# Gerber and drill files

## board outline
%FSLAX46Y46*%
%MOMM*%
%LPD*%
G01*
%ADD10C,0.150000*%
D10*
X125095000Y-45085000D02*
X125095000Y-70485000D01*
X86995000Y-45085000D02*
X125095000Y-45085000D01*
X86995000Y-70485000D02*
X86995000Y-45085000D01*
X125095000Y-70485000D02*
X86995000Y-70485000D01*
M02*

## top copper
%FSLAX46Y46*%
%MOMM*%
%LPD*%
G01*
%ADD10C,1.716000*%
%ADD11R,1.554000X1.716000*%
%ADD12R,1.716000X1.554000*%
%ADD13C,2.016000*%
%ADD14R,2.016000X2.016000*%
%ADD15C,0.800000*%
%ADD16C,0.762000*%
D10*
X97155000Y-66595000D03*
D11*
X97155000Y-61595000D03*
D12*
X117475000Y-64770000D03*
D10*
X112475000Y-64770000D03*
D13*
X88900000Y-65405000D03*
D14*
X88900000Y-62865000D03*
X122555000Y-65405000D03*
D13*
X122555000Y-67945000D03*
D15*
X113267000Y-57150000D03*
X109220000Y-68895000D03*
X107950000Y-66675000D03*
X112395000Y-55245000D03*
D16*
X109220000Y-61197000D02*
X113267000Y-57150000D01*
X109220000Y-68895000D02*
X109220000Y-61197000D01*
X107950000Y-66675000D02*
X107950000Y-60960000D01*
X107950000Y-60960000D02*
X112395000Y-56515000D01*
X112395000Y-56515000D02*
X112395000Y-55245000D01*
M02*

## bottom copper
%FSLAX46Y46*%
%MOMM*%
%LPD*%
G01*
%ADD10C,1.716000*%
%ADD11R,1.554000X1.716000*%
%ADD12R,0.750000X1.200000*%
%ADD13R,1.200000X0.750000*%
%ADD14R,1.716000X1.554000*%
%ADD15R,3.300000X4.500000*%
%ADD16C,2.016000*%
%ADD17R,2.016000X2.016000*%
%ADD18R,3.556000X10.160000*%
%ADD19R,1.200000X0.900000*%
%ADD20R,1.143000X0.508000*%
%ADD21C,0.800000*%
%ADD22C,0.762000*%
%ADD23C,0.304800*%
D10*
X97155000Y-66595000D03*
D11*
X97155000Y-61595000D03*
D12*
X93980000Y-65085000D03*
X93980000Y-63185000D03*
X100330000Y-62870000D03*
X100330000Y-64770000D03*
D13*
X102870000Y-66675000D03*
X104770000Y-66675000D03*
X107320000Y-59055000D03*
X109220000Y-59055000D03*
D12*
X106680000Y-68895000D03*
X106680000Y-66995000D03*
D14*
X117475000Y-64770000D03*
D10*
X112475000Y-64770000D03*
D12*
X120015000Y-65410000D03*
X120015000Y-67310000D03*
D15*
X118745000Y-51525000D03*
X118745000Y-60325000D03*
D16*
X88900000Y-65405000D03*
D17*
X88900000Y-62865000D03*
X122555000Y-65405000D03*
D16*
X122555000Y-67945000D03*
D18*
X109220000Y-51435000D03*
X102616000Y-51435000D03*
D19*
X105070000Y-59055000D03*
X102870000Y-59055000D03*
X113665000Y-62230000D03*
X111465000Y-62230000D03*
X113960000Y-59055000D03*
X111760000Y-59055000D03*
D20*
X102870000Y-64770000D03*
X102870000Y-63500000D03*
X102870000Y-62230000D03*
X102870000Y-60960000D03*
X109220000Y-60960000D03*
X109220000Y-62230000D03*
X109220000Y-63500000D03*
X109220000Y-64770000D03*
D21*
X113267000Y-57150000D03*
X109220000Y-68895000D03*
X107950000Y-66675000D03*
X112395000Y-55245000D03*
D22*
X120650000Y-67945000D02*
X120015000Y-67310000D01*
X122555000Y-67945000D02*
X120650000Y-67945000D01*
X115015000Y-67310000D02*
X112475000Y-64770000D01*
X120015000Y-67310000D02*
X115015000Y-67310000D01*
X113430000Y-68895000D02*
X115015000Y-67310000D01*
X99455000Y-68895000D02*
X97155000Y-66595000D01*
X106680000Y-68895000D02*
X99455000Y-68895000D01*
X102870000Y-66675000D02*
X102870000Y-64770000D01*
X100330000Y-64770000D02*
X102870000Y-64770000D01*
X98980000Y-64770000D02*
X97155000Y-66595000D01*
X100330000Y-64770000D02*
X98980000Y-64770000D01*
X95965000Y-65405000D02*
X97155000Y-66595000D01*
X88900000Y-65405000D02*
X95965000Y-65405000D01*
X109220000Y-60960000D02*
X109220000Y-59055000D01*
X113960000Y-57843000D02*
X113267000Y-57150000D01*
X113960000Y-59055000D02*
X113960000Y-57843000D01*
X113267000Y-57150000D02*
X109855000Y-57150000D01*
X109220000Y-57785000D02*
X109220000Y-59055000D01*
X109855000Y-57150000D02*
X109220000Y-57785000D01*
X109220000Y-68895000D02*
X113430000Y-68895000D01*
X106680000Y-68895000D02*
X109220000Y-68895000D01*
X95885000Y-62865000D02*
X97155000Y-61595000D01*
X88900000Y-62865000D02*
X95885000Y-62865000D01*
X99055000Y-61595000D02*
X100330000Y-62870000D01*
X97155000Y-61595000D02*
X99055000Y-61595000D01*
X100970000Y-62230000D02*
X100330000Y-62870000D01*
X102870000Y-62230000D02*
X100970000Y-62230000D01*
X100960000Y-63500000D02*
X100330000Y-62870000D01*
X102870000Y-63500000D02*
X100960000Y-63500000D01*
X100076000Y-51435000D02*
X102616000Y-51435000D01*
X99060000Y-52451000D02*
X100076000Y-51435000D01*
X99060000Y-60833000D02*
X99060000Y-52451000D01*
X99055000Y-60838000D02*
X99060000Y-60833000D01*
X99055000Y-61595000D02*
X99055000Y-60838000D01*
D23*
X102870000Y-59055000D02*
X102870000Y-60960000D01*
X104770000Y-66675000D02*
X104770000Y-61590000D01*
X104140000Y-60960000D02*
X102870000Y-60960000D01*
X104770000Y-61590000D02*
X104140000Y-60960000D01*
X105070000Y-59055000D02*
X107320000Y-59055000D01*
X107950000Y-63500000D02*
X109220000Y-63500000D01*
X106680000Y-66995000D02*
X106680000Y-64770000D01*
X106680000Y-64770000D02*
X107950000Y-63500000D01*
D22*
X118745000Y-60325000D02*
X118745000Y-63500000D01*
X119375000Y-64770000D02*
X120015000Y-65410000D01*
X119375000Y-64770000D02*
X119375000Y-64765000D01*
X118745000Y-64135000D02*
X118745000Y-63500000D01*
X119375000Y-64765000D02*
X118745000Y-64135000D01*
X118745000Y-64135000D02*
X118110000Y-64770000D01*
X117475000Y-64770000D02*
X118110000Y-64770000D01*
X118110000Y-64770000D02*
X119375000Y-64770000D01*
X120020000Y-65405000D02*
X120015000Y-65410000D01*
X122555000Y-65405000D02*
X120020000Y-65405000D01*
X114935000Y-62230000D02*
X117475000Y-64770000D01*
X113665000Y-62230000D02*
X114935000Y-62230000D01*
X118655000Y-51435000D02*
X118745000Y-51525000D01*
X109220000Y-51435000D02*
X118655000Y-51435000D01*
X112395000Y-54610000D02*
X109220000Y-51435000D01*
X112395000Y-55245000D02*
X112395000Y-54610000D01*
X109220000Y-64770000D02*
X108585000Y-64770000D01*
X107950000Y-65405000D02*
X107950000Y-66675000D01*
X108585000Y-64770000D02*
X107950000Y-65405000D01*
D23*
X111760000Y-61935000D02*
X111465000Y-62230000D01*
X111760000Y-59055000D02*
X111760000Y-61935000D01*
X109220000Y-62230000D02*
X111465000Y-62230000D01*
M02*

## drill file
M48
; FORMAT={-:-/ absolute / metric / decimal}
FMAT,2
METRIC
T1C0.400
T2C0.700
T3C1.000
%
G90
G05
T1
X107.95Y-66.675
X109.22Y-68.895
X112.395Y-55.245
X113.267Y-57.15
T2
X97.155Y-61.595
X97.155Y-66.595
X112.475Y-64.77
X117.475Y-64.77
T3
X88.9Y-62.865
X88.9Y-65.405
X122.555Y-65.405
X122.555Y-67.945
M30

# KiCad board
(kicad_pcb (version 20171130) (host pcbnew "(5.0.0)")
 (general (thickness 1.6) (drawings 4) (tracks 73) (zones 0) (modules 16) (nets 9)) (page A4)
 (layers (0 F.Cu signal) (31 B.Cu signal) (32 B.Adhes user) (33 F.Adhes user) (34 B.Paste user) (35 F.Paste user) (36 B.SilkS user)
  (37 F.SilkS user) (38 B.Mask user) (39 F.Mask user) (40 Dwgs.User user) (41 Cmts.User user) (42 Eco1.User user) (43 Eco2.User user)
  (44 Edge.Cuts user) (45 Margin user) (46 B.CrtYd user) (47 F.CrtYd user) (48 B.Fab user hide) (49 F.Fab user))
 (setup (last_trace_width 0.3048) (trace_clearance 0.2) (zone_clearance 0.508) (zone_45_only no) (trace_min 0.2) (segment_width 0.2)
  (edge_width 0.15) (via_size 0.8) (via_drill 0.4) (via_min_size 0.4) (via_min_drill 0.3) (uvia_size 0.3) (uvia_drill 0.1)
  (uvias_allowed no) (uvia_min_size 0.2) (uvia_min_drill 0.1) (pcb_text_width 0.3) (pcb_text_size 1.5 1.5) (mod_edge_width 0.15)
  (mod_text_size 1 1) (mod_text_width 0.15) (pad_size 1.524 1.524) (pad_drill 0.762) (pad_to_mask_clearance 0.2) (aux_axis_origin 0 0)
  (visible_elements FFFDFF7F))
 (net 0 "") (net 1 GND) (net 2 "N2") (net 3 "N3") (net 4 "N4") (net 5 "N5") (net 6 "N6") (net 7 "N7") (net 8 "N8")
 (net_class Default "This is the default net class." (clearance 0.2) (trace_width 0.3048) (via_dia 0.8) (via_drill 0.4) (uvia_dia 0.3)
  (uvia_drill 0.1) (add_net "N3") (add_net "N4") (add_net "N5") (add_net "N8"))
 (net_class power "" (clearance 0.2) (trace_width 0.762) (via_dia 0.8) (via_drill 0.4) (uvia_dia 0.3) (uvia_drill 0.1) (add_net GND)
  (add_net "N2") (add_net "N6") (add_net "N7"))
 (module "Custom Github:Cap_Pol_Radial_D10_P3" (layer F.Cu) (at 97.155 61.595 270)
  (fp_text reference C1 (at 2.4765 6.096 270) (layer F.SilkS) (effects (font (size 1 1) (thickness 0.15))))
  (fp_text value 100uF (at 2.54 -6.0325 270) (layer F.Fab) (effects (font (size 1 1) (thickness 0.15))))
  (pad 2 thru_hole circle (at 5 0 270) (size 1.716 1.716) (drill 0.7) (layers *.Cu *.Mask F.SilkS) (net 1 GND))
  (pad 1 thru_hole rect (at 0 0 270) (size 1.716 1.554) (drill 0.7) (layers *.Cu *.Mask F.SilkS) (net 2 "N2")))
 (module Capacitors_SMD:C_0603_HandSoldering (layer B.Cu) (at 93.98 64.135 270)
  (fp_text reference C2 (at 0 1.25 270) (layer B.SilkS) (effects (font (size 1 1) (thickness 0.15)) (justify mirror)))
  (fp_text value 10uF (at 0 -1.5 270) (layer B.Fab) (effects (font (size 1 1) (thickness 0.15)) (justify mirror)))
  (pad 2 smd rect (at 0.95 0 270) (size 1.2 0.75) (layers B.Cu B.Paste B.Mask) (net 1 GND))
  (pad 1 smd rect (at -0.95 0 270) (size 1.2 0.75) (layers B.Cu B.Paste B.Mask) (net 2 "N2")))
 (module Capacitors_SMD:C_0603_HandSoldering (layer B.Cu) (at 100.33 63.82 270)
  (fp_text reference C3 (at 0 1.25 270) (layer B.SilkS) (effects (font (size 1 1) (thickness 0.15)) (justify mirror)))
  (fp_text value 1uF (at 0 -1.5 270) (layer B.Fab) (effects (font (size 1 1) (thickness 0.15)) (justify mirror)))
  (pad 1 smd rect (at -0.95 0 270) (size 1.2 0.75) (layers B.Cu B.Paste B.Mask) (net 2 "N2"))
  (pad 2 smd rect (at 0.95 0 270) (size 1.2 0.75) (layers B.Cu B.Paste B.Mask) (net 1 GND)))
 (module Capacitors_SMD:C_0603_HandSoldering (layer B.Cu) (at 103.82 66.675 180)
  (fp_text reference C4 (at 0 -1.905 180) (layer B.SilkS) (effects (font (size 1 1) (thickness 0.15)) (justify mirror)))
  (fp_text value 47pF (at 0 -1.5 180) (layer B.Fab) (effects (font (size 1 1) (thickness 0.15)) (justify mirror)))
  (pad 2 smd rect (at 0.95 0 180) (size 1.2 0.75) (layers B.Cu B.Paste B.Mask) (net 1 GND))
  (pad 1 smd rect (at -0.95 0 180) (size 1.2 0.75) (layers B.Cu B.Paste B.Mask) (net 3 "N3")))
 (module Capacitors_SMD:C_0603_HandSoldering (layer B.Cu) (at 108.27 59.055)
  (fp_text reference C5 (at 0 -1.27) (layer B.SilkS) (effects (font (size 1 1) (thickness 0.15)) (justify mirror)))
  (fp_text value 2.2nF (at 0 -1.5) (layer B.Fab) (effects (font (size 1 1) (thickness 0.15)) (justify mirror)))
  (pad 1 smd rect (at -0.95 0) (size 1.2 0.75) (layers B.Cu B.Paste B.Mask) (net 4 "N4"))
  (pad 2 smd rect (at 0.95 0) (size 1.2 0.75) (layers B.Cu B.Paste B.Mask) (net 1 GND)))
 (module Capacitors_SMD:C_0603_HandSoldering (layer B.Cu) (at 106.68 67.945 270)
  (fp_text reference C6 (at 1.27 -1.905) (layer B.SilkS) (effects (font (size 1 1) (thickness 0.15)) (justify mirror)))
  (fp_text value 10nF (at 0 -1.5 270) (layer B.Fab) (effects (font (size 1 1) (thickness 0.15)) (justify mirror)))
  (pad 2 smd rect (at 0.95 0 270) (size 1.2 0.75) (layers B.Cu B.Paste B.Mask) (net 1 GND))
  (pad 1 smd rect (at -0.95 0 270) (size 1.2 0.75) (layers B.Cu B.Paste B.Mask) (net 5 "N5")))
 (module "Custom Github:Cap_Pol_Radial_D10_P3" (layer F.Cu) (at 117.475 64.77 180)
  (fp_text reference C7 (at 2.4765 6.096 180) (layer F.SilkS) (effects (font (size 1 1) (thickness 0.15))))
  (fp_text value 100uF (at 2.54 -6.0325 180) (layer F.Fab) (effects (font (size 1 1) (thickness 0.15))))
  (pad 1 thru_hole rect (at 0 0 180) (size 1.716 1.554) (drill 0.7) (layers *.Cu *.Mask F.SilkS) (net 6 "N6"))
  (pad 2 thru_hole circle (at 5 0 180) (size 1.716 1.716) (drill 0.7) (layers *.Cu *.Mask F.SilkS) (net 1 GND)))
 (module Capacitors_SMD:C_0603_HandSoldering (layer B.Cu) (at 120.015 66.36 270)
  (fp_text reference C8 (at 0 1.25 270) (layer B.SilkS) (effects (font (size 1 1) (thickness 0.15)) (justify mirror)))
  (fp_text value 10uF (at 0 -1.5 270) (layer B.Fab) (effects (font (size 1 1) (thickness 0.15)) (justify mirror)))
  (pad 1 smd rect (at -0.95 0 270) (size 1.2 0.75) (layers B.Cu B.Paste B.Mask) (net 6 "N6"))
  (pad 2 smd rect (at 0.95 0 270) (size 1.2 0.75) (layers B.Cu B.Paste B.Mask) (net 1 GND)))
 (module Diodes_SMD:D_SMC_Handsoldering (layer B.Cu) (at 118.745 55.925 90)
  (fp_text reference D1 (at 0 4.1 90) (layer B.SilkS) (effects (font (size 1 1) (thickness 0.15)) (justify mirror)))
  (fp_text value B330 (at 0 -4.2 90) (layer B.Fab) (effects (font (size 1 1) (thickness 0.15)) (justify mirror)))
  (pad 2 smd rect (at 4.4 0) (size 3.3 4.5) (layers B.Cu B.Paste B.Mask) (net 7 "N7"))
  (pad 1 smd rect (at -4.4 0) (size 3.3 4.5) (layers B.Cu B.Paste B.Mask) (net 6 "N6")))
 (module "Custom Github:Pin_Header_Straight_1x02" (layer F.Cu) (at 88.9 62.865)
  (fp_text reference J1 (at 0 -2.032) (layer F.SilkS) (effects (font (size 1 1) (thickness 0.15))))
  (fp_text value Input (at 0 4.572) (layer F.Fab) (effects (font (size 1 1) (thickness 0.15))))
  (pad 2 thru_hole circle (at 0 2.54) (size 2.016 2.016) (drill 1) (layers *.Cu *.Mask F.SilkS) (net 1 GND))
  (pad 1 thru_hole rect (at 0 0) (size 2.016 2.016) (drill 1) (layers *.Cu *.Mask F.SilkS) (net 2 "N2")))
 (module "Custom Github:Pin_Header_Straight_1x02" (layer F.Cu) (at 122.555 65.405)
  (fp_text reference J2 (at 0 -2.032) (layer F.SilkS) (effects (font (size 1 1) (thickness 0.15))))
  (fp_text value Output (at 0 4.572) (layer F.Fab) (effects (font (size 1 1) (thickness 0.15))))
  (pad 1 thru_hole rect (at 0 0) (size 2.016 2.016) (drill 1) (layers *.Cu *.Mask F.SilkS) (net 6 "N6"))
  (pad 2 thru_hole circle (at 0 2.54) (size 2.016 2.016) (drill 1) (layers *.Cu *.Mask F.SilkS) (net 1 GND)))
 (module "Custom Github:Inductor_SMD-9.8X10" (layer B.Cu) (at 105.918 51.435)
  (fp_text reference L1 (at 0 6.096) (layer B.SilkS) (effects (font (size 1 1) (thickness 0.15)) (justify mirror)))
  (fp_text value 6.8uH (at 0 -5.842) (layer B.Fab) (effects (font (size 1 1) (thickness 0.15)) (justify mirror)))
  (pad 2 smd rect (at 3.302 0) (size 3.556 10.16) (layers B.Cu B.Paste B.Mask) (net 7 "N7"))
  (pad 1 smd rect (at -3.302 0) (size 3.556 10.16) (layers B.Cu B.Paste B.Mask) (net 2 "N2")))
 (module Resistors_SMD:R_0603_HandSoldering (layer B.Cu) (at 103.97 59.055)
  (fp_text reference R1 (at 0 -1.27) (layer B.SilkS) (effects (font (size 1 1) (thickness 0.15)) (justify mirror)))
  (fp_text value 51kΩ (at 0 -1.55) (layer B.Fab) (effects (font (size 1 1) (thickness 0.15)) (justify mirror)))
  (pad 2 smd rect (at 1.1 0) (size 1.2 0.9) (layers B.Cu B.Paste B.Mask) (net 4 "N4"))
  (pad 1 smd rect (at -1.1 0) (size 1.2 0.9) (layers B.Cu B.Paste B.Mask) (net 3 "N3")))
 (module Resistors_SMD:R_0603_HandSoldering (layer B.Cu) (at 112.565 62.23 180)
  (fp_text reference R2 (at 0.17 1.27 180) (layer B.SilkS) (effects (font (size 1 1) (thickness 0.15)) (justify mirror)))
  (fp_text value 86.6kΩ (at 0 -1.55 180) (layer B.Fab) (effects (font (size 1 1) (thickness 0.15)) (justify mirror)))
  (pad 1 smd rect (at -1.1 0 180) (size 1.2 0.9) (layers B.Cu B.Paste B.Mask) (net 6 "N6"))
  (pad 2 smd rect (at 1.1 0 180) (size 1.2 0.9) (layers B.Cu B.Paste B.Mask) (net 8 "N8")))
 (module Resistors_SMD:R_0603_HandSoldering (layer B.Cu) (at 112.86 59.055)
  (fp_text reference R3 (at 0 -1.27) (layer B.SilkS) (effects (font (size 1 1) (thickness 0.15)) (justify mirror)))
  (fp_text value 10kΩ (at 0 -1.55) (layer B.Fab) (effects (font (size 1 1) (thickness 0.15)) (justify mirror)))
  (pad 2 smd rect (at 1.1 0) (size 1.2 0.9) (layers B.Cu B.Paste B.Mask) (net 1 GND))
  (pad 1 smd rect (at -1.1 0) (size 1.2 0.9) (layers B.Cu B.Paste B.Mask) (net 8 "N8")))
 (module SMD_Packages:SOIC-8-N (layer B.Cu) (at 106.045 62.865 90)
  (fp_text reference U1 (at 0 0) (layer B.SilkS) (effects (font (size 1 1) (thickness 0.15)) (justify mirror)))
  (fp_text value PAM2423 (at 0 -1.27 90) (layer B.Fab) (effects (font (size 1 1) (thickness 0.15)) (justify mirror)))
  (pad 1 smd rect (at -1.905 -3.175 90) (size 0.508 1.143) (layers B.Cu B.Paste B.Mask) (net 1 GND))
  (pad 2 smd rect (at -0.635 -3.175 90) (size 0.508 1.143) (layers B.Cu B.Paste B.Mask) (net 2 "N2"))
  (pad 3 smd rect (at 0.635 -3.175 90) (size 0.508 1.143) (layers B.Cu B.Paste B.Mask) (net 2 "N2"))
  (pad 4 smd rect (at 1.905 -3.175 90) (size 0.508 1.143) (layers B.Cu B.Paste B.Mask) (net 3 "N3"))
  (pad 5 smd rect (at 1.905 3.175 90) (size 0.508 1.143) (layers B.Cu B.Paste B.Mask) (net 1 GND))
  (pad 6 smd rect (at 0.635 3.175 90) (size 0.508 1.143) (layers B.Cu B.Paste B.Mask) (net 8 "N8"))
  (pad 7 smd rect (at -0.635 3.175 90) (size 0.508 1.143) (layers B.Cu B.Paste B.Mask) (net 5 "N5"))
  (pad 8 smd rect (at -1.905 3.175 90) (size 0.508 1.143) (layers B.Cu B.Paste B.Mask) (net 7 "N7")))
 (gr_line (start 125.095 45.085) (end 125.095 70.485) (layer Edge.Cuts) (width 0.15))
 (gr_line (start 86.995 45.085) (end 125.095 45.085) (layer Edge.Cuts) (width 0.15))
 (gr_line (start 86.995 70.485) (end 86.995 45.085) (layer Edge.Cuts) (width 0.15))
 (gr_line (start 125.095 70.485) (end 86.995 70.485) (layer Edge.Cuts) (width 0.15))
 (segment (start 120.65 67.945) (end 120.015 67.31) (width 0.762) (layer B.Cu) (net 1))
 (segment (start 122.555 67.945) (end 120.65 67.945) (width 0.762) (layer B.Cu) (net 1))
 (segment (start 115.015 67.31) (end 112.475 64.77) (width 0.762) (layer B.Cu) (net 1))
 (segment (start 120.015 67.31) (end 115.015 67.31) (width 0.762) (layer B.Cu) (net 1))
 (segment (start 113.43 68.895) (end 115.015 67.31) (width 0.762) (layer B.Cu) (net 1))
 (segment (start 99.455 68.895) (end 97.155 66.595) (width 0.762) (layer B.Cu) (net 1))
 (segment (start 106.68 68.895) (end 99.455 68.895) (width 0.762) (layer B.Cu) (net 1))
 (segment (start 102.87 66.675) (end 102.87 64.77) (width 0.762) (layer B.Cu) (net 1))
 (segment (start 100.33 64.77) (end 102.87 64.77) (width 0.762) (layer B.Cu) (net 1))
 (segment (start 98.98 64.77) (end 97.155 66.595) (width 0.762) (layer B.Cu) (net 1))
 (segment (start 100.33 64.77) (end 98.98 64.77) (width 0.762) (layer B.Cu) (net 1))
 (segment (start 95.965 65.405) (end 97.155 66.595) (width 0.762) (layer B.Cu) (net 1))
 (segment (start 88.9 65.405) (end 95.965 65.405) (width 0.762) (layer B.Cu) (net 1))
 (segment (start 109.22 60.96) (end 109.22 59.055) (width 0.762) (layer B.Cu) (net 1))
 (segment (start 113.96 57.843) (end 113.267 57.15) (width 0.762) (layer B.Cu) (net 1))
 (segment (start 113.96 59.055) (end 113.96 57.843) (width 0.762) (layer B.Cu) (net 1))
 (segment (start 113.267 57.15) (end 109.855 57.15) (width 0.762) (layer B.Cu) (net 1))
 (segment (start 109.22 57.785) (end 109.22 59.055) (width 0.762) (layer B.Cu) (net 1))
 (segment (start 109.855 57.15) (end 109.22 57.785) (width 0.762) (layer B.Cu) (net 1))
 (via (at 113.267 57.15) (size 0.8) (drill 0.4) (layers F.Cu B.Cu) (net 1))
 (via (at 109.22 68.895) (size 0.8) (drill 0.4) (layers F.Cu B.Cu) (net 1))
 (segment (start 109.22 68.895) (end 113.43 68.895) (width 0.762) (layer B.Cu) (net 1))
 (segment (start 106.68 68.895) (end 109.22 68.895) (width 0.762) (layer B.Cu) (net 1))
 (segment (start 109.22 61.197) (end 113.267 57.15) (width 0.762) (layer F.Cu) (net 1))
 (segment (start 109.22 68.895) (end 109.22 61.197) (width 0.762) (layer F.Cu) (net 1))
 (segment (start 95.885 62.865) (end 97.155 61.595) (width 0.762) (layer B.Cu) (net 2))
 (segment (start 88.9 62.865) (end 95.885 62.865) (width 0.762) (layer B.Cu) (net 2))
 (segment (start 99.055 61.595) (end 100.33 62.87) (width 0.762) (layer B.Cu) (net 2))
 (segment (start 97.155 61.595) (end 99.055 61.595) (width 0.762) (layer B.Cu) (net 2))
 (segment (start 100.97 62.23) (end 100.33 62.87) (width 0.762) (layer B.Cu) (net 2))
 (segment (start 102.87 62.23) (end 100.97 62.23) (width 0.762) (layer B.Cu) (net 2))
 (segment (start 100.96 63.5) (end 100.33 62.87) (width 0.762) (layer B.Cu) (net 2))
 (segment (start 102.87 63.5) (end 100.96 63.5) (width 0.762) (layer B.Cu) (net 2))
 (segment (start 100.076 51.435) (end 102.616 51.435) (width 0.762) (layer B.Cu) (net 2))
 (segment (start 99.06 52.451) (end 100.076 51.435) (width 0.762) (layer B.Cu) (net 2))
 (segment (start 99.06 60.833) (end 99.06 52.451) (width 0.762) (layer B.Cu) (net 2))
 (segment (start 99.055 60.838) (end 99.06 60.833) (width 0.762) (layer B.Cu) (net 2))
 (segment (start 99.055 61.595) (end 99.055 60.838) (width 0.762) (layer B.Cu) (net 2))
 (segment (start 102.87 59.055) (end 102.87 60.96) (width 0.3048) (layer B.Cu) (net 3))
 (segment (start 104.77 66.675) (end 104.77 61.59) (width 0.3048) (layer B.Cu) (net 3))
 (segment (start 104.14 60.96) (end 102.87 60.96) (width 0.3048) (layer B.Cu) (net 3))
 (segment (start 104.77 61.59) (end 104.14 60.96) (width 0.3048) (layer B.Cu) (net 3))
 (segment (start 105.07 59.055) (end 107.32 59.055) (width 0.3048) (layer B.Cu) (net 4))
 (segment (start 107.95 63.5) (end 109.22 63.5) (width 0.3048) (layer B.Cu) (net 5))
 (segment (start 106.68 66.995) (end 106.68 64.77) (width 0.3048) (layer B.Cu) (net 5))
 (segment (start 106.68 64.77) (end 107.95 63.5) (width 0.3048) (layer B.Cu) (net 5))
 (segment (start 118.745 60.325) (end 118.745 63.5) (width 0.762) (layer B.Cu) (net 6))
 (segment (start 119.375 64.77) (end 120.015 65.41) (width 0.762) (layer B.Cu) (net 6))
 (segment (start 119.375 64.77) (end 119.375 64.765) (width 0.762) (layer B.Cu) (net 6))
 (segment (start 118.745 64.135) (end 118.745 63.5) (width 0.762) (layer B.Cu) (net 6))
 (segment (start 119.375 64.765) (end 118.745 64.135) (width 0.762) (layer B.Cu) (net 6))
 (segment (start 118.745 64.135) (end 118.11 64.77) (width 0.762) (layer B.Cu) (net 6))
 (segment (start 117.475 64.77) (end 118.11 64.77) (width 0.762) (layer B.Cu) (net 6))
 (segment (start 118.11 64.77) (end 119.375 64.77) (width 0.762) (layer B.Cu) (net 6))
 (segment (start 120.02 65.405) (end 120.015 65.41) (width 0.762) (layer B.Cu) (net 6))
 (segment (start 122.555 65.405) (end 120.02 65.405) (width 0.762) (layer B.Cu) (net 6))
 (segment (start 114.935 62.23) (end 117.475 64.77) (width 0.762) (layer B.Cu) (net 6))
 (segment (start 113.665 62.23) (end 114.935 62.23) (width 0.762) (layer B.Cu) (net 6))
 (segment (start 118.655 51.435) (end 118.745 51.525) (width 0.762) (layer B.Cu) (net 7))
 (segment (start 109.22 51.435) (end 118.655 51.435) (width 0.762) (layer B.Cu) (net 7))
 (via (at 107.95 66.675) (size 0.8) (drill 0.4) (layers F.Cu B.Cu) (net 7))
 (segment (start 107.95 66.675) (end 107.95 60.96) (width 0.762) (layer F.Cu) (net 7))
 (via (at 112.395 55.245) (size 0.8) (drill 0.4) (layers F.Cu B.Cu) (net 7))
 (segment (start 107.95 60.96) (end 112.395 56.515) (width 0.762) (layer F.Cu) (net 7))
 (segment (start 112.395 56.515) (end 112.395 55.245) (width 0.762) (layer F.Cu) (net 7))
 (segment (start 112.395 54.61) (end 109.22 51.435) (width 0.762) (layer B.Cu) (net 7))
 (segment (start 112.395 55.245) (end 112.395 54.61) (width 0.762) (layer B.Cu) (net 7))
 (segment (start 109.22 64.77) (end 108.585 64.77) (width 0.762) (layer B.Cu) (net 7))
 (segment (start 107.95 65.405) (end 107.95 66.675) (width 0.762) (layer B.Cu) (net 7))
 (segment (start 108.585 64.77) (end 107.95 65.405) (width 0.762) (layer B.Cu) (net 7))
 (segment (start 111.76 61.935) (end 111.465 62.23) (width 0.3048) (layer B.Cu) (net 8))
 (segment (start 111.76 59.055) (end 111.76 61.935) (width 0.3048) (layer B.Cu) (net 8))
 (segment (start 109.22 62.23) (end 111.465 62.23) (width 0.3048) (layer B.Cu) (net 8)))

